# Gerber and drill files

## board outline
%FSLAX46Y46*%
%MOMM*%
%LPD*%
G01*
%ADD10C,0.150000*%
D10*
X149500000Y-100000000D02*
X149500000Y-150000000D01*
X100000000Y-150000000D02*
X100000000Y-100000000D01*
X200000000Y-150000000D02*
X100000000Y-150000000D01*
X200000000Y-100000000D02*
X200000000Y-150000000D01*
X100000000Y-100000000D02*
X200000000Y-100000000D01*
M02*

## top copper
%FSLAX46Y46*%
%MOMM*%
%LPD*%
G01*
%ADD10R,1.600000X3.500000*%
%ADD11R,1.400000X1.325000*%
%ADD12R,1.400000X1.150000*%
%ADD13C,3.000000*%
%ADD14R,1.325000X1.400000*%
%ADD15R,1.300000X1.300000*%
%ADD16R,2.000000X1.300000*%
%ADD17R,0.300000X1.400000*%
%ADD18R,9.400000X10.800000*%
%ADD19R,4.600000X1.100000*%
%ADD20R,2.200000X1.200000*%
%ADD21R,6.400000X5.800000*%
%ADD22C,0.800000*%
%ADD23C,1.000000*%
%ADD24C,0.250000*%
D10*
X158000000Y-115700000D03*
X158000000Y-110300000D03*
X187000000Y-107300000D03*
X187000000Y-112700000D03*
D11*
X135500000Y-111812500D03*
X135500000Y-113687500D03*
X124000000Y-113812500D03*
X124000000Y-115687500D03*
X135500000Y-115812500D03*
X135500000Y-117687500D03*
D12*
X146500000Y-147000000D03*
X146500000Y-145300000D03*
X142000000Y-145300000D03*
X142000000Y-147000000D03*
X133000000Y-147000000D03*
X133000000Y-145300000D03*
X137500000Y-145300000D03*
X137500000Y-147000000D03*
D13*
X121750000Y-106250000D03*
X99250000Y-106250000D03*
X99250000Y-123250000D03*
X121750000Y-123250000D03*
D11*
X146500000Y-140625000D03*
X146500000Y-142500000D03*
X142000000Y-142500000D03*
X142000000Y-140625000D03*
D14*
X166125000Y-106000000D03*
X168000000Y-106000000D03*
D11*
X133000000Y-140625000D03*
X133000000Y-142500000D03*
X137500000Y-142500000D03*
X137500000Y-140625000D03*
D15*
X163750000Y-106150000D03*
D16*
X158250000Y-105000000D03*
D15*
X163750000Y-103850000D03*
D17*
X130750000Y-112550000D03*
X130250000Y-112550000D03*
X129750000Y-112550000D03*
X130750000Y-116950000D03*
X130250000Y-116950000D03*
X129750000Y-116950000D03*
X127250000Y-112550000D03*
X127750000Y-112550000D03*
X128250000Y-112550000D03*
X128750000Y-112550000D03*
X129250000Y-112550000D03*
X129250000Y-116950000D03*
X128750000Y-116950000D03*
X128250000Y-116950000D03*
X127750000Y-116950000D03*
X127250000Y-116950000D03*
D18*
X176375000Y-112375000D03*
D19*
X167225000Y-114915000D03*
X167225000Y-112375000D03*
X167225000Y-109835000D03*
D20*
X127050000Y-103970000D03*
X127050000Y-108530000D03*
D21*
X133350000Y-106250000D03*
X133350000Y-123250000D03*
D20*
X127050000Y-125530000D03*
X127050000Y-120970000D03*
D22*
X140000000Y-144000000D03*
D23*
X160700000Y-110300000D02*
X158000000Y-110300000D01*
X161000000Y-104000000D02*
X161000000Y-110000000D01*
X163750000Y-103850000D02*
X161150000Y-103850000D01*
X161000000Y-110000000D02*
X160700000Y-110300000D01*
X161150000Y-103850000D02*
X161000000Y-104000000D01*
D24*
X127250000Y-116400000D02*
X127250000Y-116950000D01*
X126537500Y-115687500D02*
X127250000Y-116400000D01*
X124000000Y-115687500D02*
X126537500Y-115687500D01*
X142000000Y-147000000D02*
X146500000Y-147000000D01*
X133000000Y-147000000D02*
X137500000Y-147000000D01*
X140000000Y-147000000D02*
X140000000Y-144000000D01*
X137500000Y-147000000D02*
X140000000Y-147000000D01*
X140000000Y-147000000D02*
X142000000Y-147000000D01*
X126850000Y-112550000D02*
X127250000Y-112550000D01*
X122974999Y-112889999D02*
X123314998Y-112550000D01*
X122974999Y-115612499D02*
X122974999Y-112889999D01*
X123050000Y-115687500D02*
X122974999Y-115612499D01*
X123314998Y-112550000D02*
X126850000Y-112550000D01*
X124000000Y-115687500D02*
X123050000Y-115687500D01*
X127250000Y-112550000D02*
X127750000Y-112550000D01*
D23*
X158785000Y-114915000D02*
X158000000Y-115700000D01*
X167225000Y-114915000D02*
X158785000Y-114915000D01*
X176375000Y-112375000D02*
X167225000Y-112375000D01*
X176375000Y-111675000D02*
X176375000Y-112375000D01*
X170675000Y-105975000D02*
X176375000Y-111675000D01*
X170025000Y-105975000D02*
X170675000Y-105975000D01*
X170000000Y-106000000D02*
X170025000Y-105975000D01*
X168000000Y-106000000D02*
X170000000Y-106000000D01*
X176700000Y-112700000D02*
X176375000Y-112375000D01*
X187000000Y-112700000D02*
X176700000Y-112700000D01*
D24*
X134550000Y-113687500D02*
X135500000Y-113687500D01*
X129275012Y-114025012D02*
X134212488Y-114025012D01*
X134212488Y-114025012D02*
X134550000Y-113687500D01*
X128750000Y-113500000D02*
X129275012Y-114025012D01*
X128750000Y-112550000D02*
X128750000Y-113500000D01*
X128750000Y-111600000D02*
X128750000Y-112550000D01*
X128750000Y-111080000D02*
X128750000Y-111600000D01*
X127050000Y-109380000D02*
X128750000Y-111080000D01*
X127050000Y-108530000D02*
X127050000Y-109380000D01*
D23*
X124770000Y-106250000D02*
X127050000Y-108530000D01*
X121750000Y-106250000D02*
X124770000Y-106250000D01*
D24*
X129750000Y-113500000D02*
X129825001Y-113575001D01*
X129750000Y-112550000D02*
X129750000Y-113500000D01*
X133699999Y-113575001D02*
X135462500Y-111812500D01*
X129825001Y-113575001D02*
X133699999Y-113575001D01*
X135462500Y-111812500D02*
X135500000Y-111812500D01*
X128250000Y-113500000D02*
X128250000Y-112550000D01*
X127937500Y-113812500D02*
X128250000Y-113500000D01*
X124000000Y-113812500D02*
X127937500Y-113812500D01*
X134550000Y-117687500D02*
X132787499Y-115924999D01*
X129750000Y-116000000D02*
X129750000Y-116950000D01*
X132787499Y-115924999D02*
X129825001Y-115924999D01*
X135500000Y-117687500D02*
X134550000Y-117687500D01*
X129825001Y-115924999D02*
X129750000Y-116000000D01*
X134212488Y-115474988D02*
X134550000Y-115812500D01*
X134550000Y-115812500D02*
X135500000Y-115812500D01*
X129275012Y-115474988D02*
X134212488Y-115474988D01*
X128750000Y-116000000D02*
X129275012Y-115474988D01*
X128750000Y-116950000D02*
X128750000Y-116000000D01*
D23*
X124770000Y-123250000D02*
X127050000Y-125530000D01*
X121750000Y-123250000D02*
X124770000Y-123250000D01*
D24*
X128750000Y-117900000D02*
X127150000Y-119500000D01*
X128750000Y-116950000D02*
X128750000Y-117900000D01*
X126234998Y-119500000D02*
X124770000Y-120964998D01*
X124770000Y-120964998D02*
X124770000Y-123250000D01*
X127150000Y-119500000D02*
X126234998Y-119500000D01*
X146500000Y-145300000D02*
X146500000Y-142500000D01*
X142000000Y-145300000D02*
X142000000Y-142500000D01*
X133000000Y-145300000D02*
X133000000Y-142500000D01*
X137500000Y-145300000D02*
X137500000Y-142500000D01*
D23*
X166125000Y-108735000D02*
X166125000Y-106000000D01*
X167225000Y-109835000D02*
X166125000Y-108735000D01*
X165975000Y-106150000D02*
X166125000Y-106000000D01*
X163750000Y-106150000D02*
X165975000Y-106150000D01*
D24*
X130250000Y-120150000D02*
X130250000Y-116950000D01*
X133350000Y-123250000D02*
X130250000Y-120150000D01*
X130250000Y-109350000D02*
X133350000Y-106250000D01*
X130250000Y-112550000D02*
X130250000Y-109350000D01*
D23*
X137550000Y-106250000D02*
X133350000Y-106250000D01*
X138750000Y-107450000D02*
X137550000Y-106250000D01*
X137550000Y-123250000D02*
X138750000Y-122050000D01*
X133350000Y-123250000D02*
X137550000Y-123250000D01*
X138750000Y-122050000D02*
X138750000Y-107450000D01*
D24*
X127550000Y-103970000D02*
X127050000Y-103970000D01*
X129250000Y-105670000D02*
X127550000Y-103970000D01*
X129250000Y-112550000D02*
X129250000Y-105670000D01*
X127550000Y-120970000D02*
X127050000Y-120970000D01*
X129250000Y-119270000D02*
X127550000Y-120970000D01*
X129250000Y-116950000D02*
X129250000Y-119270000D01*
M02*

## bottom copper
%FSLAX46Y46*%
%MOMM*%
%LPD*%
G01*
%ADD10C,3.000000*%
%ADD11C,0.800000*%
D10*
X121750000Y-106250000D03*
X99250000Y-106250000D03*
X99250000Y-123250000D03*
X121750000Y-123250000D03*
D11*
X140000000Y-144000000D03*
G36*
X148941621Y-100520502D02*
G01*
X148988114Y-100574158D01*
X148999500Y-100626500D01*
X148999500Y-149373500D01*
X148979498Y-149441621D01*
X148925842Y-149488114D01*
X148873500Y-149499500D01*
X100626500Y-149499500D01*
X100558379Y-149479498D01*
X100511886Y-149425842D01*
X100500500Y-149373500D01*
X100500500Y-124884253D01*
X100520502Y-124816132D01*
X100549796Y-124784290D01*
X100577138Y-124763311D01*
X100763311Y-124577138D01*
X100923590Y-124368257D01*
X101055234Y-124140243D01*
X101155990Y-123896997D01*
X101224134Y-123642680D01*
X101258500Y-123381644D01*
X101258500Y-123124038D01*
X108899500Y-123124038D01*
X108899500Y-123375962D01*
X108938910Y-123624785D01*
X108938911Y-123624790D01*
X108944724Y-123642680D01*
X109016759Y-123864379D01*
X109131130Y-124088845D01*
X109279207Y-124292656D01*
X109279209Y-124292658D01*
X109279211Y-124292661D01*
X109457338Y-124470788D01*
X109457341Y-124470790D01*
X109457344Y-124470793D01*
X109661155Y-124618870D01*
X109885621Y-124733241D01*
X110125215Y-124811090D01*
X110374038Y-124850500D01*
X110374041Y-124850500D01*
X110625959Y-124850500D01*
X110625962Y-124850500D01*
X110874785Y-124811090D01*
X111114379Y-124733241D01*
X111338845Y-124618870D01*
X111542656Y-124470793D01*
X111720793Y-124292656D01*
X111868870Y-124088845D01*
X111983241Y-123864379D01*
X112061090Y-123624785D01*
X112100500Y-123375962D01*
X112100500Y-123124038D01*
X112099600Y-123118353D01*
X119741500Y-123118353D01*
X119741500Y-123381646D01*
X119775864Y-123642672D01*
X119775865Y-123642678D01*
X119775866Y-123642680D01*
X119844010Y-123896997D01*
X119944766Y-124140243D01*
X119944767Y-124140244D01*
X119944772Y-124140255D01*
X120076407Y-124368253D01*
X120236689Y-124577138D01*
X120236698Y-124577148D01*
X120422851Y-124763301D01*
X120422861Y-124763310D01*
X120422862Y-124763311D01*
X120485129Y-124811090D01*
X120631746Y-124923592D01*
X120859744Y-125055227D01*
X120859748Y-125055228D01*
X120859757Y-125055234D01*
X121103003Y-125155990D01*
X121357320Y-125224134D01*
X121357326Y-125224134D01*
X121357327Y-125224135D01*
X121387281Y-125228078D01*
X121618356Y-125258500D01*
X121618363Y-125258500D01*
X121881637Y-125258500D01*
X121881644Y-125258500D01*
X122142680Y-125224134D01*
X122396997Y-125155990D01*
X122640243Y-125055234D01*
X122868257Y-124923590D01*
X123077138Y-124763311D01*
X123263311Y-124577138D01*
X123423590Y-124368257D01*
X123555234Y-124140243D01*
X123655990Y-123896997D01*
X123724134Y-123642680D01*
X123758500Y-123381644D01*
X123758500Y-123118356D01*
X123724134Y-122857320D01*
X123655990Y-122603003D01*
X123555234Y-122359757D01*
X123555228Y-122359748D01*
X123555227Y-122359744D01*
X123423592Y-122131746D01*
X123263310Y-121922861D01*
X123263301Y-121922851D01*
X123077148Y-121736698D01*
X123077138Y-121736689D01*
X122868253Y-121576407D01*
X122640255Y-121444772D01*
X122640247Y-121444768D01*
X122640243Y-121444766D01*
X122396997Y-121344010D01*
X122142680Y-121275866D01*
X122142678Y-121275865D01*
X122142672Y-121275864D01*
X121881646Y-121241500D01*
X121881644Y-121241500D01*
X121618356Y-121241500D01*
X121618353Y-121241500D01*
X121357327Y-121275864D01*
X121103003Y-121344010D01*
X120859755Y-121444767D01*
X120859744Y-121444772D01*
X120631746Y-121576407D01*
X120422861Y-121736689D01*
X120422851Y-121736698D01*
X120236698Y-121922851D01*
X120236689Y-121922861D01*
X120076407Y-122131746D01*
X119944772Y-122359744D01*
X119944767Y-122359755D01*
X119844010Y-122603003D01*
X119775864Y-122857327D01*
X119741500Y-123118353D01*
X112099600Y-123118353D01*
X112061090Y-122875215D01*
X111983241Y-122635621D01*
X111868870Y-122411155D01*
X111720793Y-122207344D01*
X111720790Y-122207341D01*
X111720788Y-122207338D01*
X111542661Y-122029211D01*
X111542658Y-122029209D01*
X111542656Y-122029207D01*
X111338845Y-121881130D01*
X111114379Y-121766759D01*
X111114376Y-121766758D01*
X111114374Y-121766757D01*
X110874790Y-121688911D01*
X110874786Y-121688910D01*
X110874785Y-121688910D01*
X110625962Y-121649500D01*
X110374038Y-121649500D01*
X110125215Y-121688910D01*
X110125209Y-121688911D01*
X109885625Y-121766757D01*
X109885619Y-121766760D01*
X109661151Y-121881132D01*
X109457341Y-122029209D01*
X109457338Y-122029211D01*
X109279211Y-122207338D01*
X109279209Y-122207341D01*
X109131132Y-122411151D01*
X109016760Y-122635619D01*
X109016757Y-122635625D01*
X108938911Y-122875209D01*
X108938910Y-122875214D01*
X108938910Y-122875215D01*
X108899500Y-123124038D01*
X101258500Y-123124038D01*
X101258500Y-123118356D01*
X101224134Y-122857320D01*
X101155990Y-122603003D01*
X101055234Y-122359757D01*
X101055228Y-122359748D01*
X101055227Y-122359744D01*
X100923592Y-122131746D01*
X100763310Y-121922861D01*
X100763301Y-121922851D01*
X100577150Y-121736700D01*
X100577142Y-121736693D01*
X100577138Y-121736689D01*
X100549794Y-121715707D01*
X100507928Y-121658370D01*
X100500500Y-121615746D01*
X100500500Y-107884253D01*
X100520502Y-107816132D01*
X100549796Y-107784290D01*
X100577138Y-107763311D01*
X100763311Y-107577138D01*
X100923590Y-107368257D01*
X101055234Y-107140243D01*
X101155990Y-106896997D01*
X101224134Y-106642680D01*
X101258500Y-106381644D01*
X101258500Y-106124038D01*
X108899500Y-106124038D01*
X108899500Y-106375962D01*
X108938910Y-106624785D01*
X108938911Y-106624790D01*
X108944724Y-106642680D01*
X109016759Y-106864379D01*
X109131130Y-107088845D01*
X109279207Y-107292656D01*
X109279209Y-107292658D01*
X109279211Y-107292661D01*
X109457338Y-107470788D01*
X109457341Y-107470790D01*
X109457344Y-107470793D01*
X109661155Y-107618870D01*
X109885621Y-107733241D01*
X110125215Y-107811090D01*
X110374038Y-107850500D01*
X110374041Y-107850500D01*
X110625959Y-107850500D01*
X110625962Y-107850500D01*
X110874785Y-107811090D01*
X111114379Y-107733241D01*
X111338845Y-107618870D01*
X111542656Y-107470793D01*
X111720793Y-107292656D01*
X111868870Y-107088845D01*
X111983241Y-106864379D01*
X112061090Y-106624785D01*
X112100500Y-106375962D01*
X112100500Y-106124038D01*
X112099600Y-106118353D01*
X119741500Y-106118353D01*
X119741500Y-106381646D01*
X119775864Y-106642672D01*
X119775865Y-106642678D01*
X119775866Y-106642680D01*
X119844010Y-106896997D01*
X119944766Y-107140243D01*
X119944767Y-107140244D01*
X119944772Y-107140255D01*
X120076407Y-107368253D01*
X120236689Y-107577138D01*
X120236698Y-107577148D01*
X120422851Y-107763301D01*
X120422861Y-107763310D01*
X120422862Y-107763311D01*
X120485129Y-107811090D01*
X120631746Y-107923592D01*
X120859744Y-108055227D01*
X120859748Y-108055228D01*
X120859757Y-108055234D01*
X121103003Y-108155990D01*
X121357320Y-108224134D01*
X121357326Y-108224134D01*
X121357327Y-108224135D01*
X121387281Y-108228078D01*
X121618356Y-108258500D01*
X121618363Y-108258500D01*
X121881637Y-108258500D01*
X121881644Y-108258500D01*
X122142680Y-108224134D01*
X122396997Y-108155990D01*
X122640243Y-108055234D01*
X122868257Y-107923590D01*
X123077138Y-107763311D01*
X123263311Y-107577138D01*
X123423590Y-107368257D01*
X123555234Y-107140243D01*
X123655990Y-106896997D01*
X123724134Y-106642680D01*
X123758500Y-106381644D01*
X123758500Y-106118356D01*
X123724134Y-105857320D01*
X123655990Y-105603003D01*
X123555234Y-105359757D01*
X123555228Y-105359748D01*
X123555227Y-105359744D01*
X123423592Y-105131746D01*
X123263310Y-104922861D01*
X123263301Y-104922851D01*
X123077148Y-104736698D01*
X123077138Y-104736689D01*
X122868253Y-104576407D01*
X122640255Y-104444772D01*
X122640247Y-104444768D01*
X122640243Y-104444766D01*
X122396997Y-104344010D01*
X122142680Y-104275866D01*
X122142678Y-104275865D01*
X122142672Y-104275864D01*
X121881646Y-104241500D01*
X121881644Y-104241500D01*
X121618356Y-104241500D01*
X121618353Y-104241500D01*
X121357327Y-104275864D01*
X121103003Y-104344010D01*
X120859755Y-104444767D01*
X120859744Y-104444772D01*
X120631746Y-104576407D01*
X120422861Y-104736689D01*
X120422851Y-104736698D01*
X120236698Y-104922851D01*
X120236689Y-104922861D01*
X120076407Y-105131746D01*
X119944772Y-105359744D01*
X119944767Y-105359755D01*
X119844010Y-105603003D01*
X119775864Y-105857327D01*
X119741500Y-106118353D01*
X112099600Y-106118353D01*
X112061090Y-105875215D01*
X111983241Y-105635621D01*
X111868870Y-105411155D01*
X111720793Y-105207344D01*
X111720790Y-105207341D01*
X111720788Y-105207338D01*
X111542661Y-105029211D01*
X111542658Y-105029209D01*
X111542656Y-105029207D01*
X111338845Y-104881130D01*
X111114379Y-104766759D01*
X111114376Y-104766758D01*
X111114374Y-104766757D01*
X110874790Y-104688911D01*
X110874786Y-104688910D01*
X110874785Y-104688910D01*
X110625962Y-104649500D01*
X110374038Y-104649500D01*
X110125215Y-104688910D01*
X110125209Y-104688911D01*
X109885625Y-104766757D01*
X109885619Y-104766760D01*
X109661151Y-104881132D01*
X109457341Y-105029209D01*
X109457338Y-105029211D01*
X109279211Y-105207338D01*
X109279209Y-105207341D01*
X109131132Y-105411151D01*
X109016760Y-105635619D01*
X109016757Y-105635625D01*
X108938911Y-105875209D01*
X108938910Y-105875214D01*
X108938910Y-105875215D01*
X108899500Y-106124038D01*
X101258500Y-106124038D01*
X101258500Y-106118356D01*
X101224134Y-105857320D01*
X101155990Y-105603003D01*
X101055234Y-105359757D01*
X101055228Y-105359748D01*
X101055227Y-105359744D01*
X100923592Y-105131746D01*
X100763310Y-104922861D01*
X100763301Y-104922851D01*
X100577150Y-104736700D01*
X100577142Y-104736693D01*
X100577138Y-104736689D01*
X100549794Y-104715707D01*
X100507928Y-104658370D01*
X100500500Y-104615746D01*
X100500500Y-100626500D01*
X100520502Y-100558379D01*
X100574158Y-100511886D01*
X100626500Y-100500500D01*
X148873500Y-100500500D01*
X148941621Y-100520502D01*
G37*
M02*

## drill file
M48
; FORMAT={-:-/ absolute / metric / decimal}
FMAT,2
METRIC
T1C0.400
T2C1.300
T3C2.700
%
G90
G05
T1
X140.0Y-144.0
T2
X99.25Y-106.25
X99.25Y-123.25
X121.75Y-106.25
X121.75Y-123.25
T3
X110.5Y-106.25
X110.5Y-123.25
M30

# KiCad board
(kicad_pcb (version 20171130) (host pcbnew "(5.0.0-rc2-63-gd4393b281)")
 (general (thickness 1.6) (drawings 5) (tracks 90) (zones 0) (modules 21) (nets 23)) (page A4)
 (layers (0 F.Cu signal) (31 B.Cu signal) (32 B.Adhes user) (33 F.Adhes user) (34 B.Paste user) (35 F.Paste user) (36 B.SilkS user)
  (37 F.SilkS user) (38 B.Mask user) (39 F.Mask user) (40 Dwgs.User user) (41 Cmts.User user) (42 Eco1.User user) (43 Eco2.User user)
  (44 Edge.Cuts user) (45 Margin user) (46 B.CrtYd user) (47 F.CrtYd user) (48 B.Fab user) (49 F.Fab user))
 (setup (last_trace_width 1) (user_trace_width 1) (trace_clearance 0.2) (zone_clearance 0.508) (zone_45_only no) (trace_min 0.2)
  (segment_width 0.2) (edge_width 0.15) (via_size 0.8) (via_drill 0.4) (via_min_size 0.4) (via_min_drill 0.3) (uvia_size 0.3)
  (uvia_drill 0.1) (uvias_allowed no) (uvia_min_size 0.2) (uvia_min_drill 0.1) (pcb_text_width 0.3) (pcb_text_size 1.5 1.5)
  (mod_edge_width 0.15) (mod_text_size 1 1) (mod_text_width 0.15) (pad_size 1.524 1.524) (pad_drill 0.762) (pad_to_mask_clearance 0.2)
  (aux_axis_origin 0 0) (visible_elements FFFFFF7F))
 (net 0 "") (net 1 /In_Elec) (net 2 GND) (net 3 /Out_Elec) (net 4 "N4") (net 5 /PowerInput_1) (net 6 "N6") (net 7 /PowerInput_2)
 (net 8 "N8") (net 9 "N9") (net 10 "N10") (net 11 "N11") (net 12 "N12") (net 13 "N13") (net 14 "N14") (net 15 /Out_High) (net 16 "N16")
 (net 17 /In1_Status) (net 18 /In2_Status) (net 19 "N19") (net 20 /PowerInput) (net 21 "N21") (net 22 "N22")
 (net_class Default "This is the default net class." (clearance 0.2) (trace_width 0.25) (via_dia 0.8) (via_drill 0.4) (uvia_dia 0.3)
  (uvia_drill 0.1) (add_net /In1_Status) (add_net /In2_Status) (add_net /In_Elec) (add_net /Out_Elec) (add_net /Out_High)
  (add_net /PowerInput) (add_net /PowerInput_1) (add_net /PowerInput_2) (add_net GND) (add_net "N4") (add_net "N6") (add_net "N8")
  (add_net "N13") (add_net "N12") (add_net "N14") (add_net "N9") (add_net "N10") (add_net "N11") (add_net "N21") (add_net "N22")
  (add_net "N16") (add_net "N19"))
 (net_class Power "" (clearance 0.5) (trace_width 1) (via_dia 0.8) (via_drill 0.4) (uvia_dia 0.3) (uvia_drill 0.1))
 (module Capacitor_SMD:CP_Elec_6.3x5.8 (layer F.Cu) (at 158 113 90)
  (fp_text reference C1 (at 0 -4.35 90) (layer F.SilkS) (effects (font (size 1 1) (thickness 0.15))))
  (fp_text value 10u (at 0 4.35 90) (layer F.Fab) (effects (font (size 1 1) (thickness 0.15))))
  (pad 1 smd rect (at -2.7 0 90) (size 3.5 1.6) (layers F.Cu F.Paste F.Mask) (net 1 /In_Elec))
  (pad 2 smd rect (at 2.7 0 90) (size 3.5 1.6) (layers F.Cu F.Paste F.Mask) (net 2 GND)))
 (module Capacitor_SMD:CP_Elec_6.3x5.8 (layer F.Cu) (at 187 110 90)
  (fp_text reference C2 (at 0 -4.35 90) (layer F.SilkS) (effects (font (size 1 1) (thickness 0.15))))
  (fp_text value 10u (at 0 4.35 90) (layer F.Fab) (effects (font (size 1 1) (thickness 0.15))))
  (pad 2 smd rect (at 2.7 0 90) (size 3.5 1.6) (layers F.Cu F.Paste F.Mask) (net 2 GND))
  (pad 1 smd rect (at -2.7 0 90) (size 3.5 1.6) (layers F.Cu F.Paste F.Mask) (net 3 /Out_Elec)))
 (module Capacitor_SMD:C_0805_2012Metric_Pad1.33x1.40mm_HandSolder (layer F.Cu) (at 135.5 112.75 90)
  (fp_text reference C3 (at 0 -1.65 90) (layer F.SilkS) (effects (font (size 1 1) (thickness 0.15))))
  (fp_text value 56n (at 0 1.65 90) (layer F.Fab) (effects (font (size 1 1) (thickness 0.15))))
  (pad 2 smd rect (at 0.9375 0 90) (size 1.325 1.4) (layers F.Cu F.Paste F.Mask) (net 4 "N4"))
  (pad 1 smd rect (at -0.9375 0 90) (size 1.325 1.4) (layers F.Cu F.Paste F.Mask) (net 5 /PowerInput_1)))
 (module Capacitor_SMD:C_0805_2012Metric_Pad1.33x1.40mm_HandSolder (layer F.Cu) (at 124 114.75 90)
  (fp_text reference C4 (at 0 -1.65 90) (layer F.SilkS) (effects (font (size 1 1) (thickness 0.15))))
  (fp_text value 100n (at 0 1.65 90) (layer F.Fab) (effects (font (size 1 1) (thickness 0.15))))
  (pad 2 smd rect (at 0.9375 0 90) (size 1.325 1.4) (layers F.Cu F.Paste F.Mask) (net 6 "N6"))
  (pad 1 smd rect (at -0.9375 0 90) (size 1.325 1.4) (layers F.Cu F.Paste F.Mask) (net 2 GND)))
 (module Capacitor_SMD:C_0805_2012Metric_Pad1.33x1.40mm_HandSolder (layer F.Cu) (at 135.5 116.75 270)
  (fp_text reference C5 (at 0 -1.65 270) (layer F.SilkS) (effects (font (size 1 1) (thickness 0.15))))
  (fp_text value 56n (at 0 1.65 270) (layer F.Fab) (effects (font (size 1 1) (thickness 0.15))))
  (pad 1 smd rect (at -0.9375 0 270) (size 1.325 1.4) (layers F.Cu F.Paste F.Mask) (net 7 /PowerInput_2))
  (pad 2 smd rect (at 0.9375 0 270) (size 1.325 1.4) (layers F.Cu F.Paste F.Mask) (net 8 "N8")))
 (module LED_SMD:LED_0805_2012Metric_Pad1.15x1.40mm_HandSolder (layer F.Cu) (at 146.5 146.15 90)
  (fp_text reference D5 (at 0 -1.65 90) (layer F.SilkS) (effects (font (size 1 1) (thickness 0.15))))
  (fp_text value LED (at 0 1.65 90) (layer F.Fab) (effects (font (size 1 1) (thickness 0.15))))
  (pad 1 smd rect (at -0.85 0 90) (size 1.15 1.4) (layers F.Cu F.Paste F.Mask) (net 2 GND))
  (pad 2 smd rect (at 0.85 0 90) (size 1.15 1.4) (layers F.Cu F.Paste F.Mask) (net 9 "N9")))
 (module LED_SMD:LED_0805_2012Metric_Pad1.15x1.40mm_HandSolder (layer F.Cu) (at 142 146.15 90)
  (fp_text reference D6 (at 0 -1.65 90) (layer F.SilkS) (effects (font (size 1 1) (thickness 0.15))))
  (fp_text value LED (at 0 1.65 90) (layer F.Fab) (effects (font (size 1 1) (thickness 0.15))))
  (pad 2 smd rect (at 0.85 0 90) (size 1.15 1.4) (layers F.Cu F.Paste F.Mask) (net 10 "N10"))
  (pad 1 smd rect (at -0.85 0 90) (size 1.15 1.4) (layers F.Cu F.Paste F.Mask) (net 2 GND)))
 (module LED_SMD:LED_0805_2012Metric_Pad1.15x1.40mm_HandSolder (layer F.Cu) (at 133 146.15 90)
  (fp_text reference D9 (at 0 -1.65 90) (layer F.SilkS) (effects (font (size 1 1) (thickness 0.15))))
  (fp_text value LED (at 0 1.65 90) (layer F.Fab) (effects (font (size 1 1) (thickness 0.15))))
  (pad 1 smd rect (at -0.85 0 90) (size 1.15 1.4) (layers F.Cu F.Paste F.Mask) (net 2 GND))
  (pad 2 smd rect (at 0.85 0 90) (size 1.15 1.4) (layers F.Cu F.Paste F.Mask) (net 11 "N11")))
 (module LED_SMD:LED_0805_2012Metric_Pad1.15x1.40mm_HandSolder (layer F.Cu) (at 137.5 146.15 90)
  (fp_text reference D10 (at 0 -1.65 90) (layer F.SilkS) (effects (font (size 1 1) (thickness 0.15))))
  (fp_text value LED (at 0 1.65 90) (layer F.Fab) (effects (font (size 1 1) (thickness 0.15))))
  (pad 2 smd rect (at 0.85 0 90) (size 1.15 1.4) (layers F.Cu F.Paste F.Mask) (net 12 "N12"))
  (pad 1 smd rect (at -0.85 0 90) (size 1.15 1.4) (layers F.Cu F.Paste F.Mask) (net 2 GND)))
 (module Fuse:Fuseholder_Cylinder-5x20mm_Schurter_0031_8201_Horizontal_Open (layer F.Cu) (at 121.75 106.25 180)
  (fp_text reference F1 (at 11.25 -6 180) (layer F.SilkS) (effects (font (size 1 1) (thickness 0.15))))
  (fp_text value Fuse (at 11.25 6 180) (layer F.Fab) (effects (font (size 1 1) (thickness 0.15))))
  (pad 1 thru_hole circle (at 0 0 180) (size 3 3) (drill 1.3) (layers *.Cu *.Mask) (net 5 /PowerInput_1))
  (pad 2 thru_hole circle (at 22.5 0 180) (size 3 3) (drill 1.3) (layers *.Cu *.Mask) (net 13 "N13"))
  (pad "" np_thru_hole circle (at 11.25 0 180) (size 2.7 2.7) (drill 2.7) (layers *.Cu *.Mask)))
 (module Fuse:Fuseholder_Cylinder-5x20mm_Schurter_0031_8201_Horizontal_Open (layer F.Cu) (at 121.75 123.25 180)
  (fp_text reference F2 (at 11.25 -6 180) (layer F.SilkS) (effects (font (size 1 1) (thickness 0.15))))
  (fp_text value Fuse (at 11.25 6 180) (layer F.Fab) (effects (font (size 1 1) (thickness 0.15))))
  (pad "" np_thru_hole circle (at 11.25 0 180) (size 2.7 2.7) (drill 2.7) (layers *.Cu *.Mask))
  (pad 2 thru_hole circle (at 22.5 0 180) (size 3 3) (drill 1.3) (layers *.Cu *.Mask) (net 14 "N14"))
  (pad 1 thru_hole circle (at 0 0 180) (size 3 3) (drill 1.3) (layers *.Cu *.Mask) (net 7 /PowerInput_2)))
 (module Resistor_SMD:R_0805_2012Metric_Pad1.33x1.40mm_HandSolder (layer F.Cu) (at 146.5 141.5625 270)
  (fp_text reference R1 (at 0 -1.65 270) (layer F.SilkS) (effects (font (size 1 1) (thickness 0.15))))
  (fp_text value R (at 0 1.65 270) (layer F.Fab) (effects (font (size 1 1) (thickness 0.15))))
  (pad 1 smd rect (at -0.9375 0 270) (size 1.325 1.4) (layers F.Cu F.Paste F.Mask) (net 3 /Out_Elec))
  (pad 2 smd rect (at 0.9375 0 270) (size 1.325 1.4) (layers F.Cu F.Paste F.Mask) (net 9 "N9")))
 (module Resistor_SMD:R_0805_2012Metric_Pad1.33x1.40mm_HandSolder (layer F.Cu) (at 142 141.5625 270)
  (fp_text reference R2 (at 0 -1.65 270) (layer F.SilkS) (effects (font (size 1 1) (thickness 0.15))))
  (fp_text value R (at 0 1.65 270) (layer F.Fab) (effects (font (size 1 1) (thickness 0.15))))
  (pad 2 smd rect (at 0.9375 0 270) (size 1.325 1.4) (layers F.Cu F.Paste F.Mask) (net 10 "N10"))
  (pad 1 smd rect (at -0.9375 0 270) (size 1.325 1.4) (layers F.Cu F.Paste F.Mask) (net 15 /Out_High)))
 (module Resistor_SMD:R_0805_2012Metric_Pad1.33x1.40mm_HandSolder (layer F.Cu) (at 167.0625 106 180)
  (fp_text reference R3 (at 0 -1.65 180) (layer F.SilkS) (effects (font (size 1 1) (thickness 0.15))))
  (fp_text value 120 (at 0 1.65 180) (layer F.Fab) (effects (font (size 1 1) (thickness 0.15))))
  (pad 2 smd rect (at 0.9375 0 180) (size 1.325 1.4) (layers F.Cu F.Paste F.Mask) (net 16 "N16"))
  (pad 1 smd rect (at -0.9375 0 180) (size 1.325 1.4) (layers F.Cu F.Paste F.Mask) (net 3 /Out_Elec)))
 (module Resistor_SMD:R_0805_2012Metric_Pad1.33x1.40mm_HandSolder (layer F.Cu) (at 133 141.5625 270)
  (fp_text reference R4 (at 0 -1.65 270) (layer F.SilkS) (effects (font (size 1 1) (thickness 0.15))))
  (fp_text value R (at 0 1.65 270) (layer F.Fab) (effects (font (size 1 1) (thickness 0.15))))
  (pad 1 smd rect (at -0.9375 0 270) (size 1.325 1.4) (layers F.Cu F.Paste F.Mask) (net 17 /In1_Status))
  (pad 2 smd rect (at 0.9375 0 270) (size 1.325 1.4) (layers F.Cu F.Paste F.Mask) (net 11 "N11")))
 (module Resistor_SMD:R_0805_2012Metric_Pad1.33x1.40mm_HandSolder (layer F.Cu) (at 137.5 141.5625 270)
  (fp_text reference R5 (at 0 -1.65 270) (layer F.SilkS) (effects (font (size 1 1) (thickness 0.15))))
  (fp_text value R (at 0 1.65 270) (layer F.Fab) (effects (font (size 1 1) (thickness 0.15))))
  (pad 2 smd rect (at 0.9375 0 270) (size 1.325 1.4) (layers F.Cu F.Paste F.Mask) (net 12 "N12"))
  (pad 1 smd rect (at -0.9375 0 270) (size 1.325 1.4) (layers F.Cu F.Paste F.Mask) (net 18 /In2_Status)))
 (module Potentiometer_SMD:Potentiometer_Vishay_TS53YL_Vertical (layer F.Cu) (at 161 105)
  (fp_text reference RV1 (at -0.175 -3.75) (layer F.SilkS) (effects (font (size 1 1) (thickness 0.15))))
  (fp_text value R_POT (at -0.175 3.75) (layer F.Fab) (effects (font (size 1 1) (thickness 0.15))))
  (pad 3 smd rect (at 2.75 1.15) (size 1.3 1.3) (layers F.Cu F.Paste F.Mask) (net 16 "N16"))
  (pad 2 smd rect (at -2.75 0) (size 2 1.3) (layers F.Cu F.Paste F.Mask) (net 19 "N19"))
  (pad 1 smd rect (at 2.75 -1.15) (size 1.3 1.3) (layers F.Cu F.Paste F.Mask) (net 2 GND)))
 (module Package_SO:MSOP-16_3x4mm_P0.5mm (layer F.Cu) (at 129 114.75 90)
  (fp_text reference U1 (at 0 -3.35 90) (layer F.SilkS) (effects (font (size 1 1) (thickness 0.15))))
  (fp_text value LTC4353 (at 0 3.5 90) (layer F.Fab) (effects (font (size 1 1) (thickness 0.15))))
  (pad 9 smd rect (at 2.2 1.75 90) (size 1.4 0.3) (layers F.Cu F.Paste F.Mask) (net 17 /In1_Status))
  (pad 10 smd rect (at 2.2 1.25 90) (size 1.4 0.3) (layers F.Cu F.Paste F.Mask) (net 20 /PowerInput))
  (pad 11 smd rect (at 2.2 0.75 90) (size 1.4 0.3) (layers F.Cu F.Paste F.Mask) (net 4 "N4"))
  (pad 8 smd rect (at -2.2 1.75 90) (size 1.4 0.3) (layers F.Cu F.Paste F.Mask) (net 18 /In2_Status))
  (pad 7 smd rect (at -2.2 1.25 90) (size 1.4 0.3) (layers F.Cu F.Paste F.Mask) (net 20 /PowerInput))
  (pad 6 smd rect (at -2.2 0.75 90) (size 1.4 0.3) (layers F.Cu F.Paste F.Mask) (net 8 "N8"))
  (pad 16 smd rect (at 2.2 -1.75 90) (size 1.4 0.3) (layers F.Cu F.Paste F.Mask) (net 2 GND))
  (pad 15 smd rect (at 2.2 -1.25 90) (size 1.4 0.3) (layers F.Cu F.Paste F.Mask) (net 2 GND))
  (pad 14 smd rect (at 2.2 -0.75 90) (size 1.4 0.3) (layers F.Cu F.Paste F.Mask) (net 6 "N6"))
  (pad 13 smd rect (at 2.2 -0.25 90) (size 1.4 0.3) (layers F.Cu F.Paste F.Mask) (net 5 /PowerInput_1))
  (pad 12 smd rect (at 2.2 0.25 90) (size 1.4 0.3) (layers F.Cu F.Paste F.Mask) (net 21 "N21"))
  (pad 5 smd rect (at -2.2 0.25 90) (size 1.4 0.3) (layers F.Cu F.Paste F.Mask) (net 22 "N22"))
  (pad 4 smd rect (at -2.2 -0.25 90) (size 1.4 0.3) (layers F.Cu F.Paste F.Mask) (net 7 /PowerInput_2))
  (pad 3 smd rect (at -2.2 -0.75 90) (size 1.4 0.3) (layers F.Cu F.Paste F.Mask))
  (pad 2 smd rect (at -2.2 -1.25 90) (size 1.4 0.3) (layers F.Cu F.Paste F.Mask))
  (pad 1 smd rect (at -2.2 -1.75 90) (size 1.4 0.3) (layers F.Cu F.Paste F.Mask) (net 2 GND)))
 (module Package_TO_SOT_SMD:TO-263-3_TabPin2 (layer F.Cu) (at 173 112.375)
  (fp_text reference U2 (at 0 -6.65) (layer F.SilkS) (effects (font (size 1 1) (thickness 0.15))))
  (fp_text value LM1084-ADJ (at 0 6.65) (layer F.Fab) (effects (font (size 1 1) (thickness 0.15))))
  (pad "" smd rect (at 0.95 2.775) (size 4.55 5.25) (layers F.Paste))
  (pad "" smd rect (at 5.8 -2.775) (size 4.55 5.25) (layers F.Paste))
  (pad "" smd rect (at 0.95 -2.775) (size 4.55 5.25) (layers F.Paste))
  (pad "" smd rect (at 5.8 2.775) (size 4.55 5.25) (layers F.Paste))
  (pad 2 smd rect (at 3.375 0) (size 9.4 10.8) (layers F.Cu F.Mask) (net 3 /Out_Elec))
  (pad 3 smd rect (at -5.775 2.54) (size 4.6 1.1) (layers F.Cu F.Paste F.Mask) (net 1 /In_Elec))
  (pad 2 smd rect (at -5.775 0) (size 4.6 1.1) (layers F.Cu F.Paste F.Mask) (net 3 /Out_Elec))
  (pad 1 smd rect (at -5.775 -2.54) (size 4.6 1.1) (layers F.Cu F.Paste F.Mask) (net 16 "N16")))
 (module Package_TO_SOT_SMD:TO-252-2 (layer F.Cu) (at 131.25 106.25)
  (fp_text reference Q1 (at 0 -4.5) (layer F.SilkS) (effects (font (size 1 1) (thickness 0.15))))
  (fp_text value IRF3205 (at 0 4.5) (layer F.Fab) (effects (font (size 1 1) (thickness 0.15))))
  (pad 1 smd rect (at -4.2 -2.28) (size 2.2 1.2) (layers F.Cu F.Paste F.Mask) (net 21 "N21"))
  (pad 3 smd rect (at -4.2 2.28) (size 2.2 1.2) (layers F.Cu F.Paste F.Mask) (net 5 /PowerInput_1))
  (pad 2 smd rect (at 2.1 0) (size 6.4 5.8) (layers F.Cu F.Mask) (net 20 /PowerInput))
  (pad "" smd rect (at 3.775 1.525) (size 3.05 2.75) (layers F.Paste))
  (pad "" smd rect (at 0.425 -1.525) (size 3.05 2.75) (layers F.Paste))
  (pad "" smd rect (at 3.775 -1.525) (size 3.05 2.75) (layers F.Paste))
  (pad "" smd rect (at 0.425 1.525) (size 3.05 2.75) (layers F.Paste)))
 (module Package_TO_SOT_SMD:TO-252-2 (layer F.Cu) (at 131.25 123.25)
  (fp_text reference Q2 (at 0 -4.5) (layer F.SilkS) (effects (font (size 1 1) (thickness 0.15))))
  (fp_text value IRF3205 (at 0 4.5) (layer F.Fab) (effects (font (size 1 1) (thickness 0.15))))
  (pad "" smd rect (at 0.425 1.525) (size 3.05 2.75) (layers F.Paste))
  (pad "" smd rect (at 3.775 -1.525) (size 3.05 2.75) (layers F.Paste))
  (pad "" smd rect (at 0.425 -1.525) (size 3.05 2.75) (layers F.Paste))
  (pad "" smd rect (at 3.775 1.525) (size 3.05 2.75) (layers F.Paste))
  (pad 2 smd rect (at 2.1 0) (size 6.4 5.8) (layers F.Cu F.Mask) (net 20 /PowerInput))
  (pad 3 smd rect (at -4.2 2.28) (size 2.2 1.2) (layers F.Cu F.Paste F.Mask) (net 7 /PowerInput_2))
  (pad 1 smd rect (at -4.2 -2.28) (size 2.2 1.2) (layers F.Cu F.Paste F.Mask) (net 22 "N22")))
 (gr_line (start 149.5 100) (end 149.5 150) (layer Edge.Cuts) (width 0.15))
 (gr_line (start 100 150) (end 100 100) (layer Edge.Cuts) (width 0.15))
 (gr_line (start 200 150) (end 100 150) (layer Edge.Cuts) (width 0.15))
 (gr_line (start 200 100) (end 200 150) (layer Edge.Cuts) (width 0.15))
 (gr_line (start 100 100) (end 200 100) (layer Edge.Cuts) (width 0.15))
 (segment (start 160.7 110.3) (end 158 110.3) (width 1) (layer F.Cu) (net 2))
 (segment (start 161 104) (end 161 110) (width 1) (layer F.Cu) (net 2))
 (segment (start 163.75 103.85) (end 161.15 103.85) (width 1) (layer F.Cu) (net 2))
 (segment (start 161 110) (end 160.7 110.3) (width 1) (layer F.Cu) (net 2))
 (segment (start 161.15 103.85) (end 161 104) (width 1) (layer F.Cu) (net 2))
 (segment (start 127.25 116.4) (end 127.25 116.95) (width 0.25) (layer F.Cu) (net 2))
 (segment (start 126.5375 115.6875) (end 127.25 116.4) (width 0.25) (layer F.Cu) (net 2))
 (segment (start 124 115.6875) (end 126.5375 115.6875) (width 0.25) (layer F.Cu) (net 2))
 (segment (start 142 147) (end 146.5 147) (width 0.25) (layer F.Cu) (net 2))
 (segment (start 133 147) (end 137.5 147) (width 0.25) (layer F.Cu) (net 2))
 (segment (start 140 147) (end 140 144) (width 0.25) (layer F.Cu) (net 2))
 (via (at 140 144) (size 0.8) (drill 0.4) (layers F.Cu B.Cu) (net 2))
 (segment (start 137.5 147) (end 140 147) (width 0.25) (layer F.Cu) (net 2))
 (segment (start 140 147) (end 142 147) (width 0.25) (layer F.Cu) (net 2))
 (segment (start 126.85 112.55) (end 127.25 112.55) (width 0.25) (layer F.Cu) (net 2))
 (segment (start 122.974999 112.889999) (end 123.314998 112.55) (width 0.25) (layer F.Cu) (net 2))
 (segment (start 122.974999 115.612499) (end 122.974999 112.889999) (width 0.25) (layer F.Cu) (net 2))
 (segment (start 123.05 115.6875) (end 122.974999 115.612499) (width 0.25) (layer F.Cu) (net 2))
 (segment (start 123.314998 112.55) (end 126.85 112.55) (width 0.25) (layer F.Cu) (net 2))
 (segment (start 124 115.6875) (end 123.05 115.6875) (width 0.25) (layer F.Cu) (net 2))
 (segment (start 127.25 112.55) (end 127.75 112.55) (width 0.25) (layer F.Cu) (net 2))
 (segment (start 158.785 114.915) (end 158 115.7) (width 1) (layer F.Cu) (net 1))
 (segment (start 167.225 114.915) (end 158.785 114.915) (width 1) (layer F.Cu) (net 1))
 (segment (start 176.375 112.375) (end 167.225 112.375) (width 1) (layer F.Cu) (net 3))
 (segment (start 176.375 111.675) (end 176.375 112.375) (width 1) (layer F.Cu) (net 3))
 (segment (start 170.675 105.975) (end 176.375 111.675) (width 1) (layer F.Cu) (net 3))
 (segment (start 170.025 105.975) (end 170.675 105.975) (width 1) (layer F.Cu) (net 3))
 (segment (start 170 106) (end 170.025 105.975) (width 1) (layer F.Cu) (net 3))
 (segment (start 168 106) (end 170 106) (width 1) (layer F.Cu) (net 3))
 (segment (start 176.7 112.7) (end 176.375 112.375) (width 1) (layer F.Cu) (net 3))
 (segment (start 187 112.7) (end 176.7 112.7) (width 1) (layer F.Cu) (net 3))
 (segment (start 134.55 113.6875) (end 135.5 113.6875) (width 0.25) (layer F.Cu) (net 5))
 (segment (start 129.275012 114.025012) (end 134.212488 114.025012) (width 0.25) (layer F.Cu) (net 5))
 (segment (start 134.212488 114.025012) (end 134.55 113.6875) (width 0.25) (layer F.Cu) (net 5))
 (segment (start 128.75 113.5) (end 129.275012 114.025012) (width 0.25) (layer F.Cu) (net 5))
 (segment (start 128.75 112.55) (end 128.75 113.5) (width 0.25) (layer F.Cu) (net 5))
 (segment (start 128.75 111.6) (end 128.75 112.55) (width 0.25) (layer F.Cu) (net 5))
 (segment (start 128.75 111.08) (end 128.75 111.6) (width 0.25) (layer F.Cu) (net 5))
 (segment (start 127.05 109.38) (end 128.75 111.08) (width 0.25) (layer F.Cu) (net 5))
 (segment (start 127.05 108.53) (end 127.05 109.38) (width 0.25) (layer F.Cu) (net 5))
 (segment (start 124.77 106.25) (end 127.05 108.53) (width 1) (layer F.Cu) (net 5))
 (segment (start 121.75 106.25) (end 124.77 106.25) (width 1) (layer F.Cu) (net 5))
 (segment (start 129.75 113.5) (end 129.825001 113.575001) (width 0.25) (layer F.Cu) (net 4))
 (segment (start 129.75 112.55) (end 129.75 113.5) (width 0.25) (layer F.Cu) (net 4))
 (segment (start 133.699999 113.575001) (end 135.4625 111.8125) (width 0.25) (layer F.Cu) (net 4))
 (segment (start 129.825001 113.575001) (end 133.699999 113.575001) (width 0.25) (layer F.Cu) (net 4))
 (segment (start 135.4625 111.8125) (end 135.5 111.8125) (width 0.25) (layer F.Cu) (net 4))
 (segment (start 128.25 113.5) (end 128.25 112.55) (width 0.25) (layer F.Cu) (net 6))
 (segment (start 127.9375 113.8125) (end 128.25 113.5) (width 0.25) (layer F.Cu) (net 6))
 (segment (start 124 113.8125) (end 127.9375 113.8125) (width 0.25) (layer F.Cu) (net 6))
 (segment (start 134.55 117.6875) (end 132.787499 115.924999) (width 0.25) (layer F.Cu) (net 8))
 (segment (start 129.75 116) (end 129.75 116.95) (width 0.25) (layer F.Cu) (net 8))
 (segment (start 132.787499 115.924999) (end 129.825001 115.924999) (width 0.25) (layer F.Cu) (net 8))
 (segment (start 135.5 117.6875) (end 134.55 117.6875) (width 0.25) (layer F.Cu) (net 8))
 (segment (start 129.825001 115.924999) (end 129.75 116) (width 0.25) (layer F.Cu) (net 8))
 (segment (start 134.212488 115.474988) (end 134.55 115.8125) (width 0.25) (layer F.Cu) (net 7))
 (segment (start 134.55 115.8125) (end 135.5 115.8125) (width 0.25) (layer F.Cu) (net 7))
 (segment (start 129.275012 115.474988) (end 134.212488 115.474988) (width 0.25) (layer F.Cu) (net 7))
 (segment (start 128.75 116) (end 129.275012 115.474988) (width 0.25) (layer F.Cu) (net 7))
 (segment (start 128.75 116.95) (end 128.75 116) (width 0.25) (layer F.Cu) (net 7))
 (segment (start 124.77 123.25) (end 127.05 125.53) (width 1) (layer F.Cu) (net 7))
 (segment (start 121.75 123.25) (end 124.77 123.25) (width 1) (layer F.Cu) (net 7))
 (segment (start 128.75 117.9) (end 127.15 119.5) (width 0.25) (layer F.Cu) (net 7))
 (segment (start 128.75 116.95) (end 128.75 117.9) (width 0.25) (layer F.Cu) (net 7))
 (segment (start 126.234998 119.5) (end 124.77 120.964998) (width 0.25) (layer F.Cu) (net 7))
 (segment (start 124.77 120.964998) (end 124.77 123.25) (width 0.25) (layer F.Cu) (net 7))
 (segment (start 127.15 119.5) (end 126.234998 119.5) (width 0.25) (layer F.Cu) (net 7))
 (segment (start 146.5 145.3) (end 146.5 142.5) (width 0.25) (layer F.Cu) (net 9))
 (segment (start 142 145.3) (end 142 142.5) (width 0.25) (layer F.Cu) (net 10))
 (segment (start 133 145.3) (end 133 142.5) (width 0.25) (layer F.Cu) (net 11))
 (segment (start 137.5 145.3) (end 137.5 142.5) (width 0.25) (layer F.Cu) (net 12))
 (segment (start 166.125 108.735) (end 166.125 106) (width 1) (layer F.Cu) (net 16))
 (segment (start 167.225 109.835) (end 166.125 108.735) (width 1) (layer F.Cu) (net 16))
 (segment (start 165.975 106.15) (end 166.125 106) (width 1) (layer F.Cu) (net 16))
 (segment (start 163.75 106.15) (end 165.975 106.15) (width 1) (layer F.Cu) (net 16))
 (segment (start 130.25 120.15) (end 130.25 116.95) (width 0.25) (layer F.Cu) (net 20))
 (segment (start 133.35 123.25) (end 130.25 120.15) (width 0.25) (layer F.Cu) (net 20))
 (segment (start 130.25 109.35) (end 133.35 106.25) (width 0.25) (layer F.Cu) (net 20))
 (segment (start 130.25 112.55) (end 130.25 109.35) (width 0.25) (layer F.Cu) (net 20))
 (segment (start 137.55 106.25) (end 133.35 106.25) (width 1) (layer F.Cu) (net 20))
 (segment (start 138.75 107.45) (end 137.55 106.25) (width 1) (layer F.Cu) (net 20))
 (segment (start 137.55 123.25) (end 138.75 122.05) (width 1) (layer F.Cu) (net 20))
 (segment (start 133.35 123.25) (end 137.55 123.25) (width 1) (layer F.Cu) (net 20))
 (segment (start 138.75 122.05) (end 138.75 107.45) (width 1) (layer F.Cu) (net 20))
 (segment (start 127.55 103.97) (end 127.05 103.97) (width 0.25) (layer F.Cu) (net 21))
 (segment (start 129.25 105.67) (end 127.55 103.97) (width 0.25) (layer F.Cu) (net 21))
 (segment (start 129.25 112.55) (end 129.25 105.67) (width 0.25) (layer F.Cu) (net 21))
 (segment (start 127.55 120.97) (end 127.05 120.97) (width 0.25) (layer F.Cu) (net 22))
 (segment (start 129.25 119.27) (end 127.55 120.97) (width 0.25) (layer F.Cu) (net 22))
 (segment (start 129.25 116.95) (end 129.25 119.27) (width 0.25) (layer F.Cu) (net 22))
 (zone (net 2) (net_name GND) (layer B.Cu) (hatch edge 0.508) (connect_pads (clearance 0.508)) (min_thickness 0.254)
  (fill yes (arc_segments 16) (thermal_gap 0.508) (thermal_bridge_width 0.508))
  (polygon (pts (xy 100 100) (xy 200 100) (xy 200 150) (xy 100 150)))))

